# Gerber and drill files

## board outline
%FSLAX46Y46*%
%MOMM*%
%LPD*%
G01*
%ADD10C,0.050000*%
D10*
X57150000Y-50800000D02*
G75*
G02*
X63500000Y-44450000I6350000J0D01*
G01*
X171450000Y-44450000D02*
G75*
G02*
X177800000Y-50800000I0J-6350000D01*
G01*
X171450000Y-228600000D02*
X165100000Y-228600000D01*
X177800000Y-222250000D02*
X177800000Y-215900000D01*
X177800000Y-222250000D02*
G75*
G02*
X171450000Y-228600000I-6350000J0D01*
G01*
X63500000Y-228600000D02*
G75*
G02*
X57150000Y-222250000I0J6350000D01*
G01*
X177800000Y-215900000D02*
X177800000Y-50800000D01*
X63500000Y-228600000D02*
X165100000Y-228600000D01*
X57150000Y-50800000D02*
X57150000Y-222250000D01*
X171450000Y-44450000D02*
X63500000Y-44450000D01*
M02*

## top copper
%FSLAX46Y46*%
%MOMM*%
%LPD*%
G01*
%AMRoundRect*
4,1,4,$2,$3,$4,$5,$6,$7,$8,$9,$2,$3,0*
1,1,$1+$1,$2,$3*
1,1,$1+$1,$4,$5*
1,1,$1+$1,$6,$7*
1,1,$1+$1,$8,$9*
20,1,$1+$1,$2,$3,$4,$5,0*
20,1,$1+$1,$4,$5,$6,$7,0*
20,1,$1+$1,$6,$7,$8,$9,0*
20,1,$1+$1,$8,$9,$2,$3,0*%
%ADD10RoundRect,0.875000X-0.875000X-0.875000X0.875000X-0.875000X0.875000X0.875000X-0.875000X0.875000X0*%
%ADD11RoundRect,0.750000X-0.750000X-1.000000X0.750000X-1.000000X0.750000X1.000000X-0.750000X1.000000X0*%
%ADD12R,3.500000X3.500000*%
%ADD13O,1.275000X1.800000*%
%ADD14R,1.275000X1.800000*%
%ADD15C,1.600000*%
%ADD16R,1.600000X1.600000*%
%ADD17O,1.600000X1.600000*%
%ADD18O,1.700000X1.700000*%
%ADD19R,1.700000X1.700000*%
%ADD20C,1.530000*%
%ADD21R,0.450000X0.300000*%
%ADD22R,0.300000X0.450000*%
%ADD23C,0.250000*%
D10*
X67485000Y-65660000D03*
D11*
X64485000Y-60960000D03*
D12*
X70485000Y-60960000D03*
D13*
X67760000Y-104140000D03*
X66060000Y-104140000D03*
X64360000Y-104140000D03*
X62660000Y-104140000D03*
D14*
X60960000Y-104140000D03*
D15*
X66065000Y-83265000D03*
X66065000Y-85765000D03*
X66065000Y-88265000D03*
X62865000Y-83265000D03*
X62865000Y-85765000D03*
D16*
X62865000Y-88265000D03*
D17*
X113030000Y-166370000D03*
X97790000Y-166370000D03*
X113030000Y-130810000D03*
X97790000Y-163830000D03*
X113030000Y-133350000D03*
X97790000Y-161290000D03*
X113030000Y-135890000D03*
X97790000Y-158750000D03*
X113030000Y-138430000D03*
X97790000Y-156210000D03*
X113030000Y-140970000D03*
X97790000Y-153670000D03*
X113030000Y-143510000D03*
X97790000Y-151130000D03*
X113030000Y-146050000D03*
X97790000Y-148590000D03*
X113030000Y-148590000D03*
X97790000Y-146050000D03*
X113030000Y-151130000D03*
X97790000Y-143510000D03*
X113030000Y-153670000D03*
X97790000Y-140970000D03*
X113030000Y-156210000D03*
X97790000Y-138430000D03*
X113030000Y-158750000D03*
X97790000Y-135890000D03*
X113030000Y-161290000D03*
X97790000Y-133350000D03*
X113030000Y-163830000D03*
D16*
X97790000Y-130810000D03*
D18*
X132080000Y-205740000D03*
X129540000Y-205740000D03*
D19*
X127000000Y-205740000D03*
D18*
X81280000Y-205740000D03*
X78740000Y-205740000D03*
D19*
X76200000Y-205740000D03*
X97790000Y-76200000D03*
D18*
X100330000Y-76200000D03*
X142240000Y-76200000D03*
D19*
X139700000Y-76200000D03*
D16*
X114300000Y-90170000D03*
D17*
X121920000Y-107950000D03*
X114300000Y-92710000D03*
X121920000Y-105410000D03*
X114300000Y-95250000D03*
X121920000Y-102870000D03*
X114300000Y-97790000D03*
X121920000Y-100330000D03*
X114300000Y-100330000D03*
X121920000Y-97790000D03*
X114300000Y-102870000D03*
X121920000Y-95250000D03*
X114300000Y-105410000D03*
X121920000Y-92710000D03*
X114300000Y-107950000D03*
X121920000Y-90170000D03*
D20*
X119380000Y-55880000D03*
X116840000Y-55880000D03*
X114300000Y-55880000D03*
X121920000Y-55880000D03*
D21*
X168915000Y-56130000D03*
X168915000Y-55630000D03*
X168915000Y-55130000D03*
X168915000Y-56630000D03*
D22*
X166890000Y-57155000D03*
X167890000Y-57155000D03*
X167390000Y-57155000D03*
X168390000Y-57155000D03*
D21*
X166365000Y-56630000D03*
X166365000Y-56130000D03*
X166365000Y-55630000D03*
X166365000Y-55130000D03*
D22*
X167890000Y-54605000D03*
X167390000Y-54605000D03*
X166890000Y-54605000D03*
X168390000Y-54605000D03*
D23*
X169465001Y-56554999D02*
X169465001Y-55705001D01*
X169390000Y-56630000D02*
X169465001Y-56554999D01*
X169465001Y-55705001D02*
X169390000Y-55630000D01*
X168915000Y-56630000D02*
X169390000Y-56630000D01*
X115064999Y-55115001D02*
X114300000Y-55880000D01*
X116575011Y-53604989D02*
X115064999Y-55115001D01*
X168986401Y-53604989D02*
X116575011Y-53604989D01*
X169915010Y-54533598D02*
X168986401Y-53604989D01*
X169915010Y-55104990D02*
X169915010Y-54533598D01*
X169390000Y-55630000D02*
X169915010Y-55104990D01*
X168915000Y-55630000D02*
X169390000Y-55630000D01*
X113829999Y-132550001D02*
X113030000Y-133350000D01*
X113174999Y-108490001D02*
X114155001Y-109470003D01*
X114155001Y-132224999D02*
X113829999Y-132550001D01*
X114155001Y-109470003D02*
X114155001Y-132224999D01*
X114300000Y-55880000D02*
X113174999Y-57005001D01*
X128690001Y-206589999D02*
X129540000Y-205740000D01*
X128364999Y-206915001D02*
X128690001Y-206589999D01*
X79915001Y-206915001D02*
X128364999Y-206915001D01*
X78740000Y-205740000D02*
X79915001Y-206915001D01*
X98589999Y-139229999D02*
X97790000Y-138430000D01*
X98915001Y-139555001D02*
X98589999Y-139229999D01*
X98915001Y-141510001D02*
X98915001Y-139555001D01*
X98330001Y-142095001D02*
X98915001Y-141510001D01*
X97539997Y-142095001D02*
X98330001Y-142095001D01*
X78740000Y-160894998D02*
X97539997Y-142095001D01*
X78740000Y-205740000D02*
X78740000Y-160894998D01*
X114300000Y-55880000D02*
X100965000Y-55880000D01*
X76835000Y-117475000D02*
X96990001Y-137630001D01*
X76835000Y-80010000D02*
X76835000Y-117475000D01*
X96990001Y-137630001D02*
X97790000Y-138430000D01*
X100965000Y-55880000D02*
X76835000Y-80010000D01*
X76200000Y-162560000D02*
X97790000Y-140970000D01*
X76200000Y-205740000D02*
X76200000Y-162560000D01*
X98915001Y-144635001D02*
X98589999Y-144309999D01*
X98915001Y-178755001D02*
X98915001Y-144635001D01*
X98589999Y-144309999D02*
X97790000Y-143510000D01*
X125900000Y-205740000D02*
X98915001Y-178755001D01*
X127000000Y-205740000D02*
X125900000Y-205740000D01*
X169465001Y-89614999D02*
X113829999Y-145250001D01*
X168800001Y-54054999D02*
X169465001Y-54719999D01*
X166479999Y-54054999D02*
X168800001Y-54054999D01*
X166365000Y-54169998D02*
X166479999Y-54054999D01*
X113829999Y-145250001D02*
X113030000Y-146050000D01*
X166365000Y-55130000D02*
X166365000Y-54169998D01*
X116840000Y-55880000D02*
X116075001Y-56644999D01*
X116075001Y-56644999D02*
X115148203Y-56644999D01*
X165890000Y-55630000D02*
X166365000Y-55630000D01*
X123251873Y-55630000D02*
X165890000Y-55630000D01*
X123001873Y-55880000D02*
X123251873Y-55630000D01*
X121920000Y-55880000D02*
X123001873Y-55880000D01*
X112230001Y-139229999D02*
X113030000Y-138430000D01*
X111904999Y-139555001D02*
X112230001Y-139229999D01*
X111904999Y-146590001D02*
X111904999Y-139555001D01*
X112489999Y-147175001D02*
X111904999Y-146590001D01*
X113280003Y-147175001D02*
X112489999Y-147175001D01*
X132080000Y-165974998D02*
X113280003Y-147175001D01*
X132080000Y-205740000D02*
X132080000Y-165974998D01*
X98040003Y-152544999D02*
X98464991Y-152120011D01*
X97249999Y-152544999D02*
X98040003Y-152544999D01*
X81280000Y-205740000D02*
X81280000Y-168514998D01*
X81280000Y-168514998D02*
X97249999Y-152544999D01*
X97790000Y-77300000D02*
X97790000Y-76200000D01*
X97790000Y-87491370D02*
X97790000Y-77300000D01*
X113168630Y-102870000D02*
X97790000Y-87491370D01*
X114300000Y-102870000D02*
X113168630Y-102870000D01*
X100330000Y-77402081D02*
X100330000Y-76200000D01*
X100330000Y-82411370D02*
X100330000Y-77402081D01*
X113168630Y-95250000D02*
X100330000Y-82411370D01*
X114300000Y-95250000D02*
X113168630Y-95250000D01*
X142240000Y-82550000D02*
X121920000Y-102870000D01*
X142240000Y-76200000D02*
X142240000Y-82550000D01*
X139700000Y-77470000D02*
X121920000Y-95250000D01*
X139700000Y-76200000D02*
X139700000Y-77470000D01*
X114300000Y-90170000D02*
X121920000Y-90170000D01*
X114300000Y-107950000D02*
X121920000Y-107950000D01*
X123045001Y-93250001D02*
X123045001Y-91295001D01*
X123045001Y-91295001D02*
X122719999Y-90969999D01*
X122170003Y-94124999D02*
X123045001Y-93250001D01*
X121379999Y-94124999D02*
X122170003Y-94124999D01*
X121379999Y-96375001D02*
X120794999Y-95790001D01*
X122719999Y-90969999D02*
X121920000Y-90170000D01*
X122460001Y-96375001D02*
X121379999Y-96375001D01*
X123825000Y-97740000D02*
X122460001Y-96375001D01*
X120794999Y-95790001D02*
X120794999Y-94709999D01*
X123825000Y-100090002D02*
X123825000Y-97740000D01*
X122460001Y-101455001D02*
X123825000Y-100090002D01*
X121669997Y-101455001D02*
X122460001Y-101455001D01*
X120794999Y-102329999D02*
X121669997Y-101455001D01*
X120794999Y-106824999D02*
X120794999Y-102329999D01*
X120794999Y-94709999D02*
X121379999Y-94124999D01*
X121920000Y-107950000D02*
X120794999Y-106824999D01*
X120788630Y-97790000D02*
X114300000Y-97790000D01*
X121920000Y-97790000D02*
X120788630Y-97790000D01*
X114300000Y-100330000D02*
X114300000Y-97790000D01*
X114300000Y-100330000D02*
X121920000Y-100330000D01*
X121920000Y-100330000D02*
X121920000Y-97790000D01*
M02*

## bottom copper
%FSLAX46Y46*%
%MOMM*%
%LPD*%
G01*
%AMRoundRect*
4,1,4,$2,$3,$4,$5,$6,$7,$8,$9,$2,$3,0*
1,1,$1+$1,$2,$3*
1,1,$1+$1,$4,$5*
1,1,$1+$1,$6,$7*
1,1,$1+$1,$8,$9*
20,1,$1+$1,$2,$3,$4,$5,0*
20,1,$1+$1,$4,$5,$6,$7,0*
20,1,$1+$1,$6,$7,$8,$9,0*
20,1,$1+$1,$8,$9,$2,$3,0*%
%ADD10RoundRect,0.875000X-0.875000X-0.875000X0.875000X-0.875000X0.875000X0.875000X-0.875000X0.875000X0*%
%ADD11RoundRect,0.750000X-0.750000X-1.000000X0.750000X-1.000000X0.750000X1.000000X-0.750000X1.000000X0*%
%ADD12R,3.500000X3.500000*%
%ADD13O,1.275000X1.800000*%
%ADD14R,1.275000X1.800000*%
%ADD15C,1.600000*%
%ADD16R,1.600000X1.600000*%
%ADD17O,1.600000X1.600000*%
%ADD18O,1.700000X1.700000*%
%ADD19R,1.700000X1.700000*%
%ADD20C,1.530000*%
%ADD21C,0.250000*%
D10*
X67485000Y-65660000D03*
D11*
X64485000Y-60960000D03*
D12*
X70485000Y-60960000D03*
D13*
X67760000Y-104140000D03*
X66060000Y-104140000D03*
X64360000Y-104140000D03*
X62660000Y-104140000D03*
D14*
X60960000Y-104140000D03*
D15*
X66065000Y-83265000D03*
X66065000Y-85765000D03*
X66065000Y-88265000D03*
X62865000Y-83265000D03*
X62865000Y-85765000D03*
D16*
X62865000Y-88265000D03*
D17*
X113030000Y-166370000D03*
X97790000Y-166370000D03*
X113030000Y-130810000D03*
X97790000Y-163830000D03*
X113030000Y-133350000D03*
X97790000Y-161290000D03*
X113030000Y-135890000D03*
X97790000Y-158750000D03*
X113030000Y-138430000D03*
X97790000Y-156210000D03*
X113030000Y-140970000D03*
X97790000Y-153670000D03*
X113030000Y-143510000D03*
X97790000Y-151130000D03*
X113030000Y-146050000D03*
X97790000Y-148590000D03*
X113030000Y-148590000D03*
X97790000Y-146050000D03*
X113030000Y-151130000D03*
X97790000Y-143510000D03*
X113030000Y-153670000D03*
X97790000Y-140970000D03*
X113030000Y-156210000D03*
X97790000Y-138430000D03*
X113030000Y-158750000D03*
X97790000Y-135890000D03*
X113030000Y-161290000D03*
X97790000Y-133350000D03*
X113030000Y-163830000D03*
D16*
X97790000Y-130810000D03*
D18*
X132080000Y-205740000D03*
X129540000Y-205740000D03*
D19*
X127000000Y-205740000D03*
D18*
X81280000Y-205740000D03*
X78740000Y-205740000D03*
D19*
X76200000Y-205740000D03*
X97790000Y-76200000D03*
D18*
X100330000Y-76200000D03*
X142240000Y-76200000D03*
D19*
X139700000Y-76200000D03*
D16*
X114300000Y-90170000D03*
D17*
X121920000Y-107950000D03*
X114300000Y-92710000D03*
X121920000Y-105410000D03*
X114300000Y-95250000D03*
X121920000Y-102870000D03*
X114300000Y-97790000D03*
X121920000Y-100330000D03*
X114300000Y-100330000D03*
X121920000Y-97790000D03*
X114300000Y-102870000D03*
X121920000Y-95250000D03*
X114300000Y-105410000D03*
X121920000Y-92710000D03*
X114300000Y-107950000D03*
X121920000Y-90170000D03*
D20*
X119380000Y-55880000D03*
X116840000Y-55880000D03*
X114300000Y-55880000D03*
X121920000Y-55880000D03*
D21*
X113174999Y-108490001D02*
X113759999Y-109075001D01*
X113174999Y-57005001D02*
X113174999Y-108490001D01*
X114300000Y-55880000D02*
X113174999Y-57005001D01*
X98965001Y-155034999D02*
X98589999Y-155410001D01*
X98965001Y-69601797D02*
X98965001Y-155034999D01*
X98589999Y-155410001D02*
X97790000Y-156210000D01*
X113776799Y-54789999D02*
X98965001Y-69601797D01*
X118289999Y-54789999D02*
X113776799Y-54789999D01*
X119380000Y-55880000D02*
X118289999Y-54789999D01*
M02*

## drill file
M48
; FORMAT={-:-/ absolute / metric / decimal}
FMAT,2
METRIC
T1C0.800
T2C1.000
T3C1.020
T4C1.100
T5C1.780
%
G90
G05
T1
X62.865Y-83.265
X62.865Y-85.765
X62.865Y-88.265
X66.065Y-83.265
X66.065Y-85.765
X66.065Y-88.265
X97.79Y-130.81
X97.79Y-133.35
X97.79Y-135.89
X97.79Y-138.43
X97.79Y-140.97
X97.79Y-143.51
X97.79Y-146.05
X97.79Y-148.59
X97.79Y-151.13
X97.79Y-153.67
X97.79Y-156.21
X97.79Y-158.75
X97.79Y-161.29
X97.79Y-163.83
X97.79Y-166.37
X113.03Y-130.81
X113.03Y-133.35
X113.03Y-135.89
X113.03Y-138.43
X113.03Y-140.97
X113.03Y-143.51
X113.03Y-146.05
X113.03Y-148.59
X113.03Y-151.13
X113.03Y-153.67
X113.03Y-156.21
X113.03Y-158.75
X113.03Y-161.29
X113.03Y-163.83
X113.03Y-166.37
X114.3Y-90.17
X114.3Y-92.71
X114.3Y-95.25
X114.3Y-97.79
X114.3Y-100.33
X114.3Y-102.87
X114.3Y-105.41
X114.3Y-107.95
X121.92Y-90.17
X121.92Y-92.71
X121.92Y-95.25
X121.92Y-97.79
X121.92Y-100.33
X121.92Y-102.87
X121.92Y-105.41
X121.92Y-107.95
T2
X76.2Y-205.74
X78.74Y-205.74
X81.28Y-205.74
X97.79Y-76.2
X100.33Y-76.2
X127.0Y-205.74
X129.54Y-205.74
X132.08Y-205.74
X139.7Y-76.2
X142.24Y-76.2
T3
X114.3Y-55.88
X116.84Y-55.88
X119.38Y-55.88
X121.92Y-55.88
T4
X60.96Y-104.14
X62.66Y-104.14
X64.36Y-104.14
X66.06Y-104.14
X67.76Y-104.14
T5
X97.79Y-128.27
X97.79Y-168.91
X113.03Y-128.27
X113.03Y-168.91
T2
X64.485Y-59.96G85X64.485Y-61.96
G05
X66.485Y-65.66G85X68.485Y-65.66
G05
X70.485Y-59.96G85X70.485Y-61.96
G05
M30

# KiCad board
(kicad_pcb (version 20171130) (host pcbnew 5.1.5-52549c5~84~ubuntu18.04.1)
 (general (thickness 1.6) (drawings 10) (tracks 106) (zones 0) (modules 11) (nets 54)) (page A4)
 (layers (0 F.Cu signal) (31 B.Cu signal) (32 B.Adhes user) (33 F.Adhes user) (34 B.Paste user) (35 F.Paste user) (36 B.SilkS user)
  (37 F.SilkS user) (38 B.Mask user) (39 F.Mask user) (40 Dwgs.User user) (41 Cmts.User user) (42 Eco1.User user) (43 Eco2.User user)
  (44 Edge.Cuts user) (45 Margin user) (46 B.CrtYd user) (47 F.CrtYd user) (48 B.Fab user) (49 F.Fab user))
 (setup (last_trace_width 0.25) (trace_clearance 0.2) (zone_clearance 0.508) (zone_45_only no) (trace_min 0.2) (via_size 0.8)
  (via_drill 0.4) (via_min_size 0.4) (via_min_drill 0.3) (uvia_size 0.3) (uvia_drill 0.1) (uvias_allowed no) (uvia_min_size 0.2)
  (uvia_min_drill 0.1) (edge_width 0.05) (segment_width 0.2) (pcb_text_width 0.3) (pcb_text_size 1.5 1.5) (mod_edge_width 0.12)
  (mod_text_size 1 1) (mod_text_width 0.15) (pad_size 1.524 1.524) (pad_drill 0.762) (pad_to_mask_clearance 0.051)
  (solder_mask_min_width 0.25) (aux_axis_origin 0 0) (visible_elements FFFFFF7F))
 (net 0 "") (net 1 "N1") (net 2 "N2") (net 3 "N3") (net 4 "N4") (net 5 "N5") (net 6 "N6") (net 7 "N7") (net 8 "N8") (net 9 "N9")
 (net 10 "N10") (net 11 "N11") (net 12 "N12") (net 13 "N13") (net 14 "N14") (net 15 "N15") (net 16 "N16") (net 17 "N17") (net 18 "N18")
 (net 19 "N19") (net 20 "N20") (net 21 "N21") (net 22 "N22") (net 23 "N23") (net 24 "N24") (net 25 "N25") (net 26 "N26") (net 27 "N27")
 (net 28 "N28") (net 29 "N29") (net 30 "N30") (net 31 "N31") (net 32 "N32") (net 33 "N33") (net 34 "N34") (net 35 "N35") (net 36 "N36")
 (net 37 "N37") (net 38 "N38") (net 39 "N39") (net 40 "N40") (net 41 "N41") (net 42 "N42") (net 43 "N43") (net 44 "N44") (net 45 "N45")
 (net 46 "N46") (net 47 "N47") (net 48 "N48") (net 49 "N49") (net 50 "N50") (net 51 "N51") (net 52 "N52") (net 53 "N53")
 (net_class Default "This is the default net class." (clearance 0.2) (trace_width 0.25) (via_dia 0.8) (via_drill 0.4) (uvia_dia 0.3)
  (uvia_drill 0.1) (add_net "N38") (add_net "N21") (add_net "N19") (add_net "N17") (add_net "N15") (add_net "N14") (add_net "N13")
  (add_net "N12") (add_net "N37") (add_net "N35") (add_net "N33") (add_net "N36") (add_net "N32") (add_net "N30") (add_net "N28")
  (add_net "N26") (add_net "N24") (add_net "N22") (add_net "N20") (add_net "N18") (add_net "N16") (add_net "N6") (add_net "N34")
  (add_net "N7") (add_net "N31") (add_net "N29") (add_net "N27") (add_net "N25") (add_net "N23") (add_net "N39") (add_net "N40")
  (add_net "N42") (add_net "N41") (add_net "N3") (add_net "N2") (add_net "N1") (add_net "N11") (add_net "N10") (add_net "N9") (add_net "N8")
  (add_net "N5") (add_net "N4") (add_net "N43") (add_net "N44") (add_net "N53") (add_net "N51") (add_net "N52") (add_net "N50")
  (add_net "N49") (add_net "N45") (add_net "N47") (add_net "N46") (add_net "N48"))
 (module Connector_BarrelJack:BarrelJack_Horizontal (layer F.Cu) (at 70.485 60.96)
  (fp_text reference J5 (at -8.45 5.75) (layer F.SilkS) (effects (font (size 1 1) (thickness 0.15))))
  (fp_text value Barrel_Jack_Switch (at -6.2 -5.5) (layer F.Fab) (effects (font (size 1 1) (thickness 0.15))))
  (pad 3 thru_hole roundrect (at -3 4.7) (size 3.5 3.5) (drill oval 3 1) (layers *.Cu *.Mask) (roundrect_rratio 0.25) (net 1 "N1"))
  (pad 2 thru_hole roundrect (at -6 0) (size 3 3.5) (drill oval 1 3) (layers *.Cu *.Mask) (roundrect_rratio 0.25) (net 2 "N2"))
  (pad 1 thru_hole rect (at 0 0) (size 3.5 3.5) (drill oval 1 3) (layers *.Cu *.Mask) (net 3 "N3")))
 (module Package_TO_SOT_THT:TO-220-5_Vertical (layer F.Cu) (at 60.96 104.14)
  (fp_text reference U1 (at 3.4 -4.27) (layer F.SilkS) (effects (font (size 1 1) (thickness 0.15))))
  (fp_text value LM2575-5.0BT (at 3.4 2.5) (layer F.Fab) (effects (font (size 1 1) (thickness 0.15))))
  (pad 5 thru_hole oval (at 6.8 0) (size 1.275 1.8) (drill 1.1) (layers *.Cu *.Mask) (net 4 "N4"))
  (pad 4 thru_hole oval (at 5.1 0) (size 1.275 1.8) (drill 1.1) (layers *.Cu *.Mask) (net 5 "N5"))
  (pad 3 thru_hole oval (at 3.4 0) (size 1.275 1.8) (drill 1.1) (layers *.Cu *.Mask) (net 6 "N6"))
  (pad 2 thru_hole oval (at 1.7 0) (size 1.275 1.8) (drill 1.1) (layers *.Cu *.Mask) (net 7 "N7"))
  (pad 1 thru_hole rect (at 0 0) (size 1.275 1.8) (drill 1.1) (layers *.Cu *.Mask) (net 2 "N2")))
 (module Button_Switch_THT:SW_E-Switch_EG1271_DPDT (layer F.Cu) (at 62.865 88.265 90)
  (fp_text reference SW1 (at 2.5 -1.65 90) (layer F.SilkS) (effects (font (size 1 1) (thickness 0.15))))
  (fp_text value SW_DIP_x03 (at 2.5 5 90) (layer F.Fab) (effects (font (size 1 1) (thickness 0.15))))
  (pad 6 thru_hole circle (at 5 3.2 90) (size 1.6 1.6) (drill 0.8) (layers *.Cu *.Mask) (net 6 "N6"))
  (pad 5 thru_hole circle (at 2.5 3.2 90) (size 1.6 1.6) (drill 0.8) (layers *.Cu *.Mask) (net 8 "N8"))
  (pad 4 thru_hole circle (at 0 3.2 90) (size 1.6 1.6) (drill 0.8) (layers *.Cu *.Mask) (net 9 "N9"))
  (pad 3 thru_hole circle (at 5 0 90) (size 1.6 1.6) (drill 0.8) (layers *.Cu *.Mask) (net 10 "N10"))
  (pad 2 thru_hole circle (at 2.5 0 90) (size 1.6 1.6) (drill 0.8) (layers *.Cu *.Mask) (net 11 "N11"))
  (pad 1 thru_hole rect (at 0 0 90) (size 1.6 1.6) (drill 0.8) (layers *.Cu *.Mask) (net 3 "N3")))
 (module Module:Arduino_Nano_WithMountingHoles (layer F.Cu) (at 97.79 130.81)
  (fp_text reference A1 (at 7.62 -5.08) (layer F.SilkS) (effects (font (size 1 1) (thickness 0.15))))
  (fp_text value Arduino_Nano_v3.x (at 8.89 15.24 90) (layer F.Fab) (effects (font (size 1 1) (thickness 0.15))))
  (pad "" np_thru_hole circle (at 0 38.1) (size 1.78 1.78) (drill 1.78) (layers *.Cu *.Mask))
  (pad "" np_thru_hole circle (at 15.24 38.1) (size 1.78 1.78) (drill 1.78) (layers *.Cu *.Mask))
  (pad "" np_thru_hole circle (at 15.24 -2.54) (size 1.78 1.78) (drill 1.78) (layers *.Cu *.Mask))
  (pad "" np_thru_hole circle (at 0 -2.54) (size 1.78 1.78) (drill 1.78) (layers *.Cu *.Mask))
  (pad 16 thru_hole oval (at 15.24 35.56) (size 1.6 1.6) (drill 0.8) (layers *.Cu *.Mask) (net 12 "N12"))
  (pad 15 thru_hole oval (at 0 35.56) (size 1.6 1.6) (drill 0.8) (layers *.Cu *.Mask) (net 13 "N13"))
  (pad 30 thru_hole oval (at 15.24 0) (size 1.6 1.6) (drill 0.8) (layers *.Cu *.Mask) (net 7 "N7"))
  (pad 14 thru_hole oval (at 0 33.02) (size 1.6 1.6) (drill 0.8) (layers *.Cu *.Mask) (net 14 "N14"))
  (pad 29 thru_hole oval (at 15.24 2.54) (size 1.6 1.6) (drill 0.8) (layers *.Cu *.Mask) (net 6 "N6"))
  (pad 13 thru_hole oval (at 0 30.48) (size 1.6 1.6) (drill 0.8) (layers *.Cu *.Mask) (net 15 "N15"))
  (pad 28 thru_hole oval (at 15.24 5.08) (size 1.6 1.6) (drill 0.8) (layers *.Cu *.Mask) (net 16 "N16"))
  (pad 12 thru_hole oval (at 0 27.94) (size 1.6 1.6) (drill 0.8) (layers *.Cu *.Mask) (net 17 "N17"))
  (pad 27 thru_hole oval (at 15.24 7.62) (size 1.6 1.6) (drill 0.8) (layers *.Cu *.Mask) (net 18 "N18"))
  (pad 11 thru_hole oval (at 0 25.4) (size 1.6 1.6) (drill 0.8) (layers *.Cu *.Mask) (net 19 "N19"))
  (pad 26 thru_hole oval (at 15.24 10.16) (size 1.6 1.6) (drill 0.8) (layers *.Cu *.Mask) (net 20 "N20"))
  (pad 10 thru_hole oval (at 0 22.86) (size 1.6 1.6) (drill 0.8) (layers *.Cu *.Mask) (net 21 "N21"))
  (pad 25 thru_hole oval (at 15.24 12.7) (size 1.6 1.6) (drill 0.8) (layers *.Cu *.Mask) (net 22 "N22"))
  (pad 9 thru_hole oval (at 0 20.32) (size 1.6 1.6) (drill 0.8) (layers *.Cu *.Mask) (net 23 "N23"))
  (pad 24 thru_hole oval (at 15.24 15.24) (size 1.6 1.6) (drill 0.8) (layers *.Cu *.Mask) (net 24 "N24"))
  (pad 8 thru_hole oval (at 0 17.78) (size 1.6 1.6) (drill 0.8) (layers *.Cu *.Mask) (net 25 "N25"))
  (pad 23 thru_hole oval (at 15.24 17.78) (size 1.6 1.6) (drill 0.8) (layers *.Cu *.Mask) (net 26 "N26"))
  (pad 7 thru_hole oval (at 0 15.24) (size 1.6 1.6) (drill 0.8) (layers *.Cu *.Mask) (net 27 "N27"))
  (pad 22 thru_hole oval (at 15.24 20.32) (size 1.6 1.6) (drill 0.8) (layers *.Cu *.Mask) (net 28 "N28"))
  (pad 6 thru_hole oval (at 0 12.7) (size 1.6 1.6) (drill 0.8) (layers *.Cu *.Mask) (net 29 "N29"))
  (pad 21 thru_hole oval (at 15.24 22.86) (size 1.6 1.6) (drill 0.8) (layers *.Cu *.Mask) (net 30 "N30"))
  (pad 5 thru_hole oval (at 0 10.16) (size 1.6 1.6) (drill 0.8) (layers *.Cu *.Mask) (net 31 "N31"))
  (pad 20 thru_hole oval (at 15.24 25.4) (size 1.6 1.6) (drill 0.8) (layers *.Cu *.Mask) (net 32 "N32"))
  (pad 4 thru_hole oval (at 0 7.62) (size 1.6 1.6) (drill 0.8) (layers *.Cu *.Mask) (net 6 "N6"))
  (pad 19 thru_hole oval (at 15.24 27.94) (size 1.6 1.6) (drill 0.8) (layers *.Cu *.Mask) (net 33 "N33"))
  (pad 3 thru_hole oval (at 0 5.08) (size 1.6 1.6) (drill 0.8) (layers *.Cu *.Mask) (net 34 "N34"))
  (pad 18 thru_hole oval (at 15.24 30.48) (size 1.6 1.6) (drill 0.8) (layers *.Cu *.Mask) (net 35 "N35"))
  (pad 2 thru_hole oval (at 0 2.54) (size 1.6 1.6) (drill 0.8) (layers *.Cu *.Mask) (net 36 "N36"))
  (pad 17 thru_hole oval (at 15.24 33.02) (size 1.6 1.6) (drill 0.8) (layers *.Cu *.Mask) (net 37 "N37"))
  (pad 1 thru_hole rect (at 0 0) (size 1.6 1.6) (drill 0.8) (layers *.Cu *.Mask) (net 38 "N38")))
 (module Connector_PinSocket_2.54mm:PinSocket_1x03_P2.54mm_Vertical (layer F.Cu) (at 127 205.74 90)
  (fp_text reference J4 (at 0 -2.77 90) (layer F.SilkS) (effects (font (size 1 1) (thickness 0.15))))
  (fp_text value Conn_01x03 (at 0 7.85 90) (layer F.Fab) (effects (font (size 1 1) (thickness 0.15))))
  (pad 3 thru_hole oval (at 0 5.08 90) (size 1.7 1.7) (drill 1) (layers *.Cu *.Mask) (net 18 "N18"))
  (pad 2 thru_hole oval (at 0 2.54 90) (size 1.7 1.7) (drill 1) (layers *.Cu *.Mask) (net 6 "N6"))
  (pad 1 thru_hole rect (at 0 0 90) (size 1.7 1.7) (drill 1) (layers *.Cu *.Mask) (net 29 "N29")))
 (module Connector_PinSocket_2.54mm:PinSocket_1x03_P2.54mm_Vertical (layer F.Cu) (at 76.2 205.74 90)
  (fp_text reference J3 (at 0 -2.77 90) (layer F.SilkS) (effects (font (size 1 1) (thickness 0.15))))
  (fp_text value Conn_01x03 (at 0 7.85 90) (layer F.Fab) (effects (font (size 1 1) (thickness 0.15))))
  (pad 3 thru_hole oval (at 0 5.08 90) (size 1.7 1.7) (drill 1) (layers *.Cu *.Mask) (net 18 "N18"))
  (pad 2 thru_hole oval (at 0 2.54 90) (size 1.7 1.7) (drill 1) (layers *.Cu *.Mask) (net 6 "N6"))
  (pad 1 thru_hole rect (at 0 0 90) (size 1.7 1.7) (drill 1) (layers *.Cu *.Mask) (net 31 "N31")))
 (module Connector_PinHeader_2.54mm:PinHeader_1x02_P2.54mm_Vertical (layer F.Cu) (at 97.79 76.2 90)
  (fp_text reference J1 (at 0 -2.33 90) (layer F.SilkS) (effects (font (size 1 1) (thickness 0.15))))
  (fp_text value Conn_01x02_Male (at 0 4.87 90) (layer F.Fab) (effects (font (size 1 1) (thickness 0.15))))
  (pad 1 thru_hole rect (at 0 0 90) (size 1.7 1.7) (drill 1) (layers *.Cu *.Mask) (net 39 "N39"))
  (pad 2 thru_hole oval (at 0 2.54 90) (size 1.7 1.7) (drill 1) (layers *.Cu *.Mask) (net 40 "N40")))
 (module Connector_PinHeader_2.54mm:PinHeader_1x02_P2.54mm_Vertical (layer F.Cu) (at 139.7 76.2 90)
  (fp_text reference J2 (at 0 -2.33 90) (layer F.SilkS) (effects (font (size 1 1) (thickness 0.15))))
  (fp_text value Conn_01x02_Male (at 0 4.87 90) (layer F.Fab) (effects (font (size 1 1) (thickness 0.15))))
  (pad 2 thru_hole oval (at 0 2.54 90) (size 1.7 1.7) (drill 1) (layers *.Cu *.Mask) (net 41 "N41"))
  (pad 1 thru_hole rect (at 0 0 90) (size 1.7 1.7) (drill 1) (layers *.Cu *.Mask) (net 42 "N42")))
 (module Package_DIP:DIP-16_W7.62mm (layer F.Cu) (at 114.3 90.17)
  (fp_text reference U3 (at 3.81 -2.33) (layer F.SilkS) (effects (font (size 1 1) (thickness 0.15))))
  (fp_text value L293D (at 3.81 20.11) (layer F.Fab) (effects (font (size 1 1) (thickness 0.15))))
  (pad 1 thru_hole rect (at 0 0) (size 1.6 1.6) (drill 0.8) (layers *.Cu *.Mask) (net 2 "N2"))
  (pad 9 thru_hole oval (at 7.62 17.78) (size 1.6 1.6) (drill 0.8) (layers *.Cu *.Mask) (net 2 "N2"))
  (pad 2 thru_hole oval (at 0 2.54) (size 1.6 1.6) (drill 0.8) (layers *.Cu *.Mask) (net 14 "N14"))
  (pad 10 thru_hole oval (at 7.62 15.24) (size 1.6 1.6) (drill 0.8) (layers *.Cu *.Mask) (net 17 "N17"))
  (pad 3 thru_hole oval (at 0 5.08) (size 1.6 1.6) (drill 0.8) (layers *.Cu *.Mask) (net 40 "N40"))
  (pad 11 thru_hole oval (at 7.62 12.7) (size 1.6 1.6) (drill 0.8) (layers *.Cu *.Mask) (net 41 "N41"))
  (pad 4 thru_hole oval (at 0 7.62) (size 1.6 1.6) (drill 0.8) (layers *.Cu *.Mask) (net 6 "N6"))
  (pad 12 thru_hole oval (at 7.62 10.16) (size 1.6 1.6) (drill 0.8) (layers *.Cu *.Mask) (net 6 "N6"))
  (pad 5 thru_hole oval (at 0 10.16) (size 1.6 1.6) (drill 0.8) (layers *.Cu *.Mask) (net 6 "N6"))
  (pad 13 thru_hole oval (at 7.62 7.62) (size 1.6 1.6) (drill 0.8) (layers *.Cu *.Mask) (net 6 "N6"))
  (pad 6 thru_hole oval (at 0 12.7) (size 1.6 1.6) (drill 0.8) (layers *.Cu *.Mask) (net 39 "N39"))
  (pad 14 thru_hole oval (at 7.62 5.08) (size 1.6 1.6) (drill 0.8) (layers *.Cu *.Mask) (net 42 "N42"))
  (pad 7 thru_hole oval (at 0 15.24) (size 1.6 1.6) (drill 0.8) (layers *.Cu *.Mask) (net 15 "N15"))
  (pad 15 thru_hole oval (at 7.62 2.54) (size 1.6 1.6) (drill 0.8) (layers *.Cu *.Mask) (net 23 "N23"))
  (pad 8 thru_hole oval (at 0 17.78) (size 1.6 1.6) (drill 0.8) (layers *.Cu *.Mask) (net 2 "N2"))
  (pad 16 thru_hole oval (at 7.62 0) (size 1.6 1.6) (drill 0.8) (layers *.Cu *.Mask) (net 2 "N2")))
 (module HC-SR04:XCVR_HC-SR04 (layer F.Cu) (at 118.11 55.88 180)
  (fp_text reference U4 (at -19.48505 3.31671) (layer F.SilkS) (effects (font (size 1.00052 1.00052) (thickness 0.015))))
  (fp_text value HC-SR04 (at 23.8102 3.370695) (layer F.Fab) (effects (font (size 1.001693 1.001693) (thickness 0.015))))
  (pad 2 thru_hole circle (at -1.27 0 180) (size 1.53 1.53) (drill 1.02) (layers *.Cu *.Mask) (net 19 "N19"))
  (pad 3 thru_hole circle (at 1.27 0 180) (size 1.53 1.53) (drill 1.02) (layers *.Cu *.Mask) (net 21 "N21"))
  (pad 4 thru_hole circle (at 3.81 0 180) (size 1.53 1.53) (drill 1.02) (layers *.Cu *.Mask) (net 6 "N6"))
  (pad 1 thru_hole circle (at -3.81 0 180) (size 1.53 1.53) (drill 1.02) (layers *.Cu *.Mask) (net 18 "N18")))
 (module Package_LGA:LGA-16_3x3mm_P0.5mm (layer F.Cu) (at 167.64 55.88)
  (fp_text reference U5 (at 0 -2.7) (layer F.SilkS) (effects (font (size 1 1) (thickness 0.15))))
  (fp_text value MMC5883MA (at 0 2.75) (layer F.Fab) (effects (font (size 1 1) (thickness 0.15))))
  (pad 10 smd rect (at 1.275 0.25 90) (size 0.3 0.45) (layers F.Cu F.Paste F.Mask) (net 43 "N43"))
  (pad 11 smd rect (at 1.275 -0.25 90) (size 0.3 0.45) (layers F.Cu F.Paste F.Mask) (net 6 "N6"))
  (pad 12 smd rect (at 1.275 -0.75 90) (size 0.3 0.45) (layers F.Cu F.Paste F.Mask) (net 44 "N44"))
  (pad 9 smd rect (at 1.275 0.75 90) (size 0.3 0.45) (layers F.Cu F.Paste F.Mask) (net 6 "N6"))
  (pad 5 smd rect (at -0.75 1.275) (size 0.3 0.45) (layers F.Cu F.Paste F.Mask) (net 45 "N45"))
  (pad 7 smd rect (at 0.25 1.275) (size 0.3 0.45) (layers F.Cu F.Paste F.Mask) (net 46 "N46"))
  (pad 6 smd rect (at -0.25 1.275) (size 0.3 0.45) (layers F.Cu F.Paste F.Mask) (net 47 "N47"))
  (pad 8 smd rect (at 0.75 1.275) (size 0.3 0.45) (layers F.Cu F.Paste F.Mask) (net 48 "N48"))
  (pad 4 smd rect (at -1.275 0.75 90) (size 0.3 0.45) (layers F.Cu F.Paste F.Mask) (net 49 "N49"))
  (pad 3 smd rect (at -1.275 0.25 90) (size 0.3 0.45) (layers F.Cu F.Paste F.Mask) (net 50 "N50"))
  (pad 2 smd rect (at -1.275 -0.25 90) (size 0.3 0.45) (layers F.Cu F.Paste F.Mask) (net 18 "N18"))
  (pad 1 smd rect (at -1.275 -0.75 90) (size 0.3 0.45) (layers F.Cu F.Paste F.Mask) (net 24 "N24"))
  (pad 14 smd rect (at 0.25 -1.275) (size 0.3 0.45) (layers F.Cu F.Paste F.Mask) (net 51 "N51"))
  (pad 15 smd rect (at -0.25 -1.275) (size 0.3 0.45) (layers F.Cu F.Paste F.Mask) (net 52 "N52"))
  (pad 16 smd rect (at -0.75 -1.275) (size 0.3 0.45) (layers F.Cu F.Paste F.Mask) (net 26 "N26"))
  (pad 13 smd rect (at 0.75 -1.275) (size 0.3 0.45) (layers F.Cu F.Paste F.Mask) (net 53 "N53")))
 (gr_arc (start 63.5 50.8) (end 63.5 44.45) (angle -90) (layer Edge.Cuts) (width 0.05))
 (gr_arc (start 171.45 50.8) (end 177.8 50.8) (angle -90) (layer Edge.Cuts) (width 0.05))
 (gr_line (start 171.45 228.6) (end 165.1 228.6) (layer Edge.Cuts) (width 0.05))
 (gr_line (start 177.8 222.25) (end 177.8 215.9) (layer Edge.Cuts) (width 0.05))
 (gr_arc (start 171.45 222.25) (end 171.45 228.6) (angle -90) (layer Edge.Cuts) (width 0.05))
 (gr_arc (start 63.5 222.25) (end 57.15 222.25) (angle -90) (layer Edge.Cuts) (width 0.05))
 (gr_line (start 177.8 215.9) (end 177.8 50.8) (layer Edge.Cuts) (width 0.05))
 (gr_line (start 63.5 228.6) (end 165.1 228.6) (layer Edge.Cuts) (width 0.05))
 (gr_line (start 57.15 50.8) (end 57.15 222.25) (layer Edge.Cuts) (width 0.05))
 (gr_line (start 171.45 44.45) (end 63.5 44.45) (layer Edge.Cuts) (width 0.05))
 (segment (start 169.465001 56.554999) (end 169.465001 55.705001) (width 0.25) (layer F.Cu) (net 6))
 (segment (start 169.39 56.63) (end 169.465001 56.554999) (width 0.25) (layer F.Cu) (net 6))
 (segment (start 169.465001 55.705001) (end 169.39 55.63) (width 0.25) (layer F.Cu) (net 6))
 (segment (start 168.915 56.63) (end 169.39 56.63) (width 0.25) (layer F.Cu) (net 6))
 (segment (start 115.064999 55.115001) (end 114.3 55.88) (width 0.25) (layer F.Cu) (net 6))
 (segment (start 116.575011 53.604989) (end 115.064999 55.115001) (width 0.25) (layer F.Cu) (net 6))
 (segment (start 168.986401 53.604989) (end 116.575011 53.604989) (width 0.25) (layer F.Cu) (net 6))
 (segment (start 169.91501 54.533598) (end 168.986401 53.604989) (width 0.25) (layer F.Cu) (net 6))
 (segment (start 169.91501 55.10499) (end 169.91501 54.533598) (width 0.25) (layer F.Cu) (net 6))
 (segment (start 169.39 55.63) (end 169.91501 55.10499) (width 0.25) (layer F.Cu) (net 6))
 (segment (start 168.915 55.63) (end 169.39 55.63) (width 0.25) (layer F.Cu) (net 6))
 (segment (start 113.829999 132.550001) (end 113.03 133.35) (width 0.25) (layer F.Cu) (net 6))
 (segment (start 113.174999 108.490001) (end 114.155001 109.470003) (width 0.25) (layer F.Cu) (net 6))
 (segment (start 114.155001 132.224999) (end 113.829999 132.550001) (width 0.25) (layer F.Cu) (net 6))
 (segment (start 114.155001 109.470003) (end 114.155001 132.224999) (width 0.25) (layer F.Cu) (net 6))
 (segment (start 114.3 55.88) (end 113.174999 57.005001) (width 0.25) (layer F.Cu) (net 6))
 (segment (start 128.690001 206.589999) (end 129.54 205.74) (width 0.25) (layer F.Cu) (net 6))
 (segment (start 128.364999 206.915001) (end 128.690001 206.589999) (width 0.25) (layer F.Cu) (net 6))
 (segment (start 79.915001 206.915001) (end 128.364999 206.915001) (width 0.25) (layer F.Cu) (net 6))
 (segment (start 78.74 205.74) (end 79.915001 206.915001) (width 0.25) (layer F.Cu) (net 6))
 (segment (start 98.589999 139.229999) (end 97.79 138.43) (width 0.25) (layer F.Cu) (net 6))
 (segment (start 98.915001 139.555001) (end 98.589999 139.229999) (width 0.25) (layer F.Cu) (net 6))
 (segment (start 98.915001 141.510001) (end 98.915001 139.555001) (width 0.25) (layer F.Cu) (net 6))
 (segment (start 98.330001 142.095001) (end 98.915001 141.510001) (width 0.25) (layer F.Cu) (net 6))
 (segment (start 97.539997 142.095001) (end 98.330001 142.095001) (width 0.25) (layer F.Cu) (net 6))
 (segment (start 78.74 160.894998) (end 97.539997 142.095001) (width 0.25) (layer F.Cu) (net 6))
 (segment (start 78.74 205.74) (end 78.74 160.894998) (width 0.25) (layer F.Cu) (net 6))
 (segment (start 114.3 55.88) (end 100.965 55.88) (width 0.25) (layer F.Cu) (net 6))
 (segment (start 76.835 117.475) (end 96.990001 137.630001) (width 0.25) (layer F.Cu) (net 6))
 (segment (start 76.835 80.01) (end 76.835 117.475) (width 0.25) (layer F.Cu) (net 6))
 (segment (start 96.990001 137.630001) (end 97.79 138.43) (width 0.25) (layer F.Cu) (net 6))
 (segment (start 100.965 55.88) (end 76.835 80.01) (width 0.25) (layer F.Cu) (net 6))
 (segment (start 113.174999 108.490001) (end 113.759999 109.075001) (width 0.25) (layer B.Cu) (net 6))
 (segment (start 113.174999 57.005001) (end 113.174999 108.490001) (width 0.25) (layer B.Cu) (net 6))
 (segment (start 114.3 55.88) (end 113.174999 57.005001) (width 0.25) (layer B.Cu) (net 6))
 (segment (start 76.2 162.56) (end 97.79 140.97) (width 0.25) (layer F.Cu) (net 31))
 (segment (start 76.2 205.74) (end 76.2 162.56) (width 0.25) (layer F.Cu) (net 31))
 (segment (start 98.915001 144.635001) (end 98.589999 144.309999) (width 0.25) (layer F.Cu) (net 29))
 (segment (start 98.915001 178.755001) (end 98.915001 144.635001) (width 0.25) (layer F.Cu) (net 29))
 (segment (start 98.589999 144.309999) (end 97.79 143.51) (width 0.25) (layer F.Cu) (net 29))
 (segment (start 125.9 205.74) (end 98.915001 178.755001) (width 0.25) (layer F.Cu) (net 29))
 (segment (start 127 205.74) (end 125.9 205.74) (width 0.25) (layer F.Cu) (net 29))
 (segment (start 169.465001 89.614999) (end 113.829999 145.250001) (width 0.25) (layer F.Cu) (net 24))
 (segment (start 168.800001 54.054999) (end 169.465001 54.719999) (width 0.25) (layer F.Cu) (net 24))
 (segment (start 166.479999 54.054999) (end 168.800001 54.054999) (width 0.25) (layer F.Cu) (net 24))
 (segment (start 166.365 54.169998) (end 166.479999 54.054999) (width 0.25) (layer F.Cu) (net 24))
 (segment (start 113.829999 145.250001) (end 113.03 146.05) (width 0.25) (layer F.Cu) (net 24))
 (segment (start 166.365 55.13) (end 166.365 54.169998) (width 0.25) (layer F.Cu) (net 24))
 (segment (start 116.84 55.88) (end 116.075001 56.644999) (width 0.25) (layer F.Cu) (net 21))
 (segment (start 116.075001 56.644999) (end 115.148203 56.644999) (width 0.25) (layer F.Cu) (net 21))
 (segment (start 98.965001 155.034999) (end 98.589999 155.410001) (width 0.25) (layer B.Cu) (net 19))
 (segment (start 98.965001 69.601797) (end 98.965001 155.034999) (width 0.25) (layer B.Cu) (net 19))
 (segment (start 98.589999 155.410001) (end 97.79 156.21) (width 0.25) (layer B.Cu) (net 19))
 (segment (start 113.776799 54.789999) (end 98.965001 69.601797) (width 0.25) (layer B.Cu) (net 19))
 (segment (start 118.289999 54.789999) (end 113.776799 54.789999) (width 0.25) (layer B.Cu) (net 19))
 (segment (start 119.38 55.88) (end 118.289999 54.789999) (width 0.25) (layer B.Cu) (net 19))
 (segment (start 165.89 55.63) (end 166.365 55.63) (width 0.25) (layer F.Cu) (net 18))
 (segment (start 123.251873 55.63) (end 165.89 55.63) (width 0.25) (layer F.Cu) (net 18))
 (segment (start 123.001873 55.88) (end 123.251873 55.63) (width 0.25) (layer F.Cu) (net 18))
 (segment (start 121.92 55.88) (end 123.001873 55.88) (width 0.25) (layer F.Cu) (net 18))
 (segment (start 112.230001 139.229999) (end 113.03 138.43) (width 0.25) (layer F.Cu) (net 18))
 (segment (start 111.904999 139.555001) (end 112.230001 139.229999) (width 0.25) (layer F.Cu) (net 18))
 (segment (start 111.904999 146.590001) (end 111.904999 139.555001) (width 0.25) (layer F.Cu) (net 18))
 (segment (start 112.489999 147.175001) (end 111.904999 146.590001) (width 0.25) (layer F.Cu) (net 18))
 (segment (start 113.280003 147.175001) (end 112.489999 147.175001) (width 0.25) (layer F.Cu) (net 18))
 (segment (start 132.08 165.974998) (end 113.280003 147.175001) (width 0.25) (layer F.Cu) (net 18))
 (segment (start 132.08 205.74) (end 132.08 165.974998) (width 0.25) (layer F.Cu) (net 18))
 (segment (start 98.040003 152.544999) (end 98.464991 152.120011) (width 0.25) (layer F.Cu) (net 18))
 (segment (start 97.249999 152.544999) (end 98.040003 152.544999) (width 0.25) (layer F.Cu) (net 18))
 (segment (start 81.28 205.74) (end 81.28 168.514998) (width 0.25) (layer F.Cu) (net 18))
 (segment (start 81.28 168.514998) (end 97.249999 152.544999) (width 0.25) (layer F.Cu) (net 18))
 (segment (start 97.79 77.3) (end 97.79 76.2) (width 0.25) (layer F.Cu) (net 39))
 (segment (start 97.79 87.49137) (end 97.79 77.3) (width 0.25) (layer F.Cu) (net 39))
 (segment (start 113.16863 102.87) (end 97.79 87.49137) (width 0.25) (layer F.Cu) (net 39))
 (segment (start 114.3 102.87) (end 113.16863 102.87) (width 0.25) (layer F.Cu) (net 39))
 (segment (start 100.33 77.402081) (end 100.33 76.2) (width 0.25) (layer F.Cu) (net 40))
 (segment (start 100.33 82.41137) (end 100.33 77.402081) (width 0.25) (layer F.Cu) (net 40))
 (segment (start 113.16863 95.25) (end 100.33 82.41137) (width 0.25) (layer F.Cu) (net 40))
 (segment (start 114.3 95.25) (end 113.16863 95.25) (width 0.25) (layer F.Cu) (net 40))
 (segment (start 142.24 82.55) (end 121.92 102.87) (width 0.25) (layer F.Cu) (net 41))
 (segment (start 142.24 76.2) (end 142.24 82.55) (width 0.25) (layer F.Cu) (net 41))
 (segment (start 139.7 77.47) (end 121.92 95.25) (width 0.25) (layer F.Cu) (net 42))
 (segment (start 139.7 76.2) (end 139.7 77.47) (width 0.25) (layer F.Cu) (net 42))
 (segment (start 114.3 90.17) (end 121.92 90.17) (width 0.25) (layer F.Cu) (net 2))
 (segment (start 114.3 107.95) (end 121.92 107.95) (width 0.25) (layer F.Cu) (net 2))
 (segment (start 123.045001 93.250001) (end 123.045001 91.295001) (width 0.25) (layer F.Cu) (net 2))
 (segment (start 123.045001 91.295001) (end 122.719999 90.969999) (width 0.25) (layer F.Cu) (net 2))
 (segment (start 122.170003 94.124999) (end 123.045001 93.250001) (width 0.25) (layer F.Cu) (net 2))
 (segment (start 121.379999 94.124999) (end 122.170003 94.124999) (width 0.25) (layer F.Cu) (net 2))
 (segment (start 121.379999 96.375001) (end 120.794999 95.790001) (width 0.25) (layer F.Cu) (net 2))
 (segment (start 122.719999 90.969999) (end 121.92 90.17) (width 0.25) (layer F.Cu) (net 2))
 (segment (start 122.460001 96.375001) (end 121.379999 96.375001) (width 0.25) (layer F.Cu) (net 2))
 (segment (start 123.825 97.74) (end 122.460001 96.375001) (width 0.25) (layer F.Cu) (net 2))
 (segment (start 120.794999 95.790001) (end 120.794999 94.709999) (width 0.25) (layer F.Cu) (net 2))
 (segment (start 123.825 100.090002) (end 123.825 97.74) (width 0.25) (layer F.Cu) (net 2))
 (segment (start 122.460001 101.455001) (end 123.825 100.090002) (width 0.25) (layer F.Cu) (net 2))
 (segment (start 121.669997 101.455001) (end 122.460001 101.455001) (width 0.25) (layer F.Cu) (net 2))
 (segment (start 120.794999 102.329999) (end 121.669997 101.455001) (width 0.25) (layer F.Cu) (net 2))
 (segment (start 120.794999 106.824999) (end 120.794999 102.329999) (width 0.25) (layer F.Cu) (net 2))
 (segment (start 120.794999 94.709999) (end 121.379999 94.124999) (width 0.25) (layer F.Cu) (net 2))
 (segment (start 121.92 107.95) (end 120.794999 106.824999) (width 0.25) (layer F.Cu) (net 2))
 (segment (start 120.78863 97.79) (end 114.3 97.79) (width 0.25) (layer F.Cu) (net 6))
 (segment (start 121.92 97.79) (end 120.78863 97.79) (width 0.25) (layer F.Cu) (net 6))
 (segment (start 114.3 100.33) (end 114.3 97.79) (width 0.25) (layer F.Cu) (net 6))
 (segment (start 114.3 100.33) (end 121.92 100.33) (width 0.25) (layer F.Cu) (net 6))
 (segment (start 121.92 100.33) (end 121.92 97.79) (width 0.25) (layer F.Cu) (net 6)))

